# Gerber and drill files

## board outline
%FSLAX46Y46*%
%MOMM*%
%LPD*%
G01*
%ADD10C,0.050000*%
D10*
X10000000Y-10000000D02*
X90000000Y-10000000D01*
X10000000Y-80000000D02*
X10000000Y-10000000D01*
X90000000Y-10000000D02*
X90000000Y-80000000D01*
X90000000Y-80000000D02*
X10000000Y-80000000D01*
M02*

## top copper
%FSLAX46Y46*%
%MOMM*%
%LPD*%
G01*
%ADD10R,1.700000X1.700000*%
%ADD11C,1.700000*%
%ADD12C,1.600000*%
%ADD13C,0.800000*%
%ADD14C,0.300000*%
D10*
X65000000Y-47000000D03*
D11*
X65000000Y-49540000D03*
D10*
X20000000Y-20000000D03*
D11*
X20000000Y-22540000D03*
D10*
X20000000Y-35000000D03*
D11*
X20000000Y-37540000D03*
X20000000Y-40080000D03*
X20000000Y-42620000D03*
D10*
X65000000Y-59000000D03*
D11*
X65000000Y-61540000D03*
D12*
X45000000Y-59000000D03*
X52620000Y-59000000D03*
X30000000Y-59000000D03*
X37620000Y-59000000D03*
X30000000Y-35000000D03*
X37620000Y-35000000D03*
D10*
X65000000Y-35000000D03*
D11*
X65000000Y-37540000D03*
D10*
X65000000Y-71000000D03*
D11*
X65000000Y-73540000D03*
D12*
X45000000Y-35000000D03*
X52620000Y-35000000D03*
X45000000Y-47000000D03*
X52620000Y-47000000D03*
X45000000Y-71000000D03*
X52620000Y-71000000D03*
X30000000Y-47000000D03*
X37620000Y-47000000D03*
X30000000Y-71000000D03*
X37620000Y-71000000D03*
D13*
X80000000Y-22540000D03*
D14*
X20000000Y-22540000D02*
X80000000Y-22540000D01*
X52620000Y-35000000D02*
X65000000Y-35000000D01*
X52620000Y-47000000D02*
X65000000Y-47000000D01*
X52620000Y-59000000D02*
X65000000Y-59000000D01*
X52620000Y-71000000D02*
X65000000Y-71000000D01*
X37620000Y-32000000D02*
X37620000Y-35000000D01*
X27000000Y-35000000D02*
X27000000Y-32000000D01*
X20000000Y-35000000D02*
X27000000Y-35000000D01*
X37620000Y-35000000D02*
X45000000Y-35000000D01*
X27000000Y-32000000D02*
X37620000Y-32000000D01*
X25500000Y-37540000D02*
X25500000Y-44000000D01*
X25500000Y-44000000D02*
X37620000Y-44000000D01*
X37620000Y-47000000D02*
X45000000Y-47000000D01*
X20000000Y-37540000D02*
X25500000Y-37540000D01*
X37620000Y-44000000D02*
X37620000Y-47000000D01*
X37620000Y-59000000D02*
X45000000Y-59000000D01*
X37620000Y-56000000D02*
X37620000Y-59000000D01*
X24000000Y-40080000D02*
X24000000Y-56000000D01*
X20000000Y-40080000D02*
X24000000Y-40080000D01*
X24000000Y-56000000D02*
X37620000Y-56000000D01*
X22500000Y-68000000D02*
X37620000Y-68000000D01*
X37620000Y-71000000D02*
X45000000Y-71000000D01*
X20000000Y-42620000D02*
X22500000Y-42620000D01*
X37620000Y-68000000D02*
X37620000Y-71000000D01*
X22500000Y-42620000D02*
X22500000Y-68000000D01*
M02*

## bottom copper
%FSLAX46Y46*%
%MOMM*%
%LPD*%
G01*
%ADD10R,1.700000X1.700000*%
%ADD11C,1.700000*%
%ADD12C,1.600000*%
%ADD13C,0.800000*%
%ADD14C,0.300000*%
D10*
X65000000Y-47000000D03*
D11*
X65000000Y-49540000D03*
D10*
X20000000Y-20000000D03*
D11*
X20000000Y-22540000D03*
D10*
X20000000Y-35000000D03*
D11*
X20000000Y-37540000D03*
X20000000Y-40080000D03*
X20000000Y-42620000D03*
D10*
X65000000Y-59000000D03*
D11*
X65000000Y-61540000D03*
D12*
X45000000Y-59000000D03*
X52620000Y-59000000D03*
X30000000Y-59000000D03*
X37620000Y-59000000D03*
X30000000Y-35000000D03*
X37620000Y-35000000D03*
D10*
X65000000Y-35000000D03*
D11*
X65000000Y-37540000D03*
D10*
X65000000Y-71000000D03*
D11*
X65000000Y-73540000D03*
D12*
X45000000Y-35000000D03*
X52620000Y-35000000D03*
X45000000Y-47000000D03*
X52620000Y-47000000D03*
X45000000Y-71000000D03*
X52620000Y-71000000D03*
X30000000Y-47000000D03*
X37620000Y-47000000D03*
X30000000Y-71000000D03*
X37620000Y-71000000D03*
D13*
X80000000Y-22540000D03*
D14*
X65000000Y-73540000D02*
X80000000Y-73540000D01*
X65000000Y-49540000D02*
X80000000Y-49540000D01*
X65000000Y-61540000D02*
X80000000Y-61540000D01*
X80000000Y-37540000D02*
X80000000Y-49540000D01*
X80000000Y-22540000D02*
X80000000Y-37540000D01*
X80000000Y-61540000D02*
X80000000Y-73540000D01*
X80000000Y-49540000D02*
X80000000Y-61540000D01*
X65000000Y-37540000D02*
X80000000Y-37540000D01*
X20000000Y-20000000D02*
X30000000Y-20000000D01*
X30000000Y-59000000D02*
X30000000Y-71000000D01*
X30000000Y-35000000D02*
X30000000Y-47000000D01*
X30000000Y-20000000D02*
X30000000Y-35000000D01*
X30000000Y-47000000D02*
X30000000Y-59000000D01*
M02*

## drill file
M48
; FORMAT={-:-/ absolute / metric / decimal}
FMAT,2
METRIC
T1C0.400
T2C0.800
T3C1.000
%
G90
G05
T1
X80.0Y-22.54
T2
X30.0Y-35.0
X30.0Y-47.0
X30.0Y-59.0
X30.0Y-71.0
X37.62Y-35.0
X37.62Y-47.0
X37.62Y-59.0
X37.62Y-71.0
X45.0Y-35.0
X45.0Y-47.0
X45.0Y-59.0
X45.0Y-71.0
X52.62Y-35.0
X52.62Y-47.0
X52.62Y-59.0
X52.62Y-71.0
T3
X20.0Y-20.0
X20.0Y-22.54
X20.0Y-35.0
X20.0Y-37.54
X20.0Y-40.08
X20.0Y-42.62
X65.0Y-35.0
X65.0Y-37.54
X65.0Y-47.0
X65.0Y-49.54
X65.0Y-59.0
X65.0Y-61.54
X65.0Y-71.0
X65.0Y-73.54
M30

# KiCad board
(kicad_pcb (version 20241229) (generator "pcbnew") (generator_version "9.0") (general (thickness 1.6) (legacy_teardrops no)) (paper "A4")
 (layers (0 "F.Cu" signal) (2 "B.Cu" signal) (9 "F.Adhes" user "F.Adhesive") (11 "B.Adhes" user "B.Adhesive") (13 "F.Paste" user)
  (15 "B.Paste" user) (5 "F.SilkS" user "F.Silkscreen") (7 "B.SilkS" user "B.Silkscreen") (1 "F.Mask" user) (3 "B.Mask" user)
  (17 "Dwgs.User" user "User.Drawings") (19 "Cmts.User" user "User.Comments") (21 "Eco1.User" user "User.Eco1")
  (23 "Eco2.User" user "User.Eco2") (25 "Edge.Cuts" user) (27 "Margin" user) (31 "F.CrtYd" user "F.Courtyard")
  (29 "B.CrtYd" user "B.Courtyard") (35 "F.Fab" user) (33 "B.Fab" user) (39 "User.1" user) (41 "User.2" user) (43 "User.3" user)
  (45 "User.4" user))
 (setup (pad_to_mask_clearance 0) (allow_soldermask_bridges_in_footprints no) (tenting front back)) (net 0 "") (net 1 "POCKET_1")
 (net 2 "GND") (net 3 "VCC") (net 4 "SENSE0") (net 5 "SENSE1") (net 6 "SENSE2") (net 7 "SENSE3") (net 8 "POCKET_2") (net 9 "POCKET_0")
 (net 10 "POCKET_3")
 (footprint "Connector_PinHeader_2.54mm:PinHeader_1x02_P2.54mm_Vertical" (layer "F.Cu") (at 65 47)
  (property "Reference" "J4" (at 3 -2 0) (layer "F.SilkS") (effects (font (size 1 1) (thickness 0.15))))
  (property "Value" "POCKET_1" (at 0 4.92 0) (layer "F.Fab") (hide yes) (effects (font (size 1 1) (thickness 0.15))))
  (pad "1" thru_hole rect (at 0 0) (size 1.7 1.7) (drill 1) (layers "*.Cu" "*.Mask") (remove_unused_layers no) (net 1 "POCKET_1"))
  (pad "2" thru_hole circle (at 0 2.54) (size 1.7 1.7) (drill 1) (layers "*.Cu" "*.Mask") (remove_unused_layers no) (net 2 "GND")))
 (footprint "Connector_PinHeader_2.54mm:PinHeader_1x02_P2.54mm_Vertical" (layer "F.Cu") (at 20 20)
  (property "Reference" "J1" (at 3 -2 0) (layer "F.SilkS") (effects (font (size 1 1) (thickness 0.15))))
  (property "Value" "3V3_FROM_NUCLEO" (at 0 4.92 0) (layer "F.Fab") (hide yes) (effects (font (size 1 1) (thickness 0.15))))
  (pad "1" thru_hole rect (at 0 0) (size 1.7 1.7) (drill 1) (layers "*.Cu" "*.Mask") (remove_unused_layers no) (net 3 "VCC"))
  (pad "2" thru_hole circle (at 0 2.54) (size 1.7 1.7) (drill 1) (layers "*.Cu" "*.Mask") (remove_unused_layers no) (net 2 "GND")))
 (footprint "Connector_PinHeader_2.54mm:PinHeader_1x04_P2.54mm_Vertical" (layer "F.Cu") (at 20 35)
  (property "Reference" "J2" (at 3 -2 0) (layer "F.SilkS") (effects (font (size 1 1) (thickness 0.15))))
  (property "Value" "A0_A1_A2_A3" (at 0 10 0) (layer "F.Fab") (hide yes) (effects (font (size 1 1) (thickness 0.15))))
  (pad "1" thru_hole rect (at 0 0) (size 1.7 1.7) (drill 1) (layers "*.Cu" "*.Mask") (remove_unused_layers no) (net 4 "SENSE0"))
  (pad "2" thru_hole circle (at 0 2.54) (size 1.7 1.7) (drill 1) (layers "*.Cu" "*.Mask") (remove_unused_layers no) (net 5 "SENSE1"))
  (pad "3" thru_hole circle (at 0 5.08) (size 1.7 1.7) (drill 1) (layers "*.Cu" "*.Mask") (remove_unused_layers no) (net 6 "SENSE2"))
  (pad "4" thru_hole circle (at 0 7.62) (size 1.7 1.7) (drill 1) (layers "*.Cu" "*.Mask") (remove_unused_layers no) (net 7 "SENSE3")))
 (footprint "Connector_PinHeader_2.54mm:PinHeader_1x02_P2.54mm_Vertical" (layer "F.Cu") (at 65 59)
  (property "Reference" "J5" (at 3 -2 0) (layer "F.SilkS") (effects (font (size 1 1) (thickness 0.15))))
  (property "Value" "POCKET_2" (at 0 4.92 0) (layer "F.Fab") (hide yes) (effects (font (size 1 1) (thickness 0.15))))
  (pad "1" thru_hole rect (at 0 0) (size 1.7 1.7) (drill 1) (layers "*.Cu" "*.Mask") (remove_unused_layers no) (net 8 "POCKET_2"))
  (pad "2" thru_hole circle (at 0 2.54) (size 1.7 1.7) (drill 1) (layers "*.Cu" "*.Mask") (remove_unused_layers no) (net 2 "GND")))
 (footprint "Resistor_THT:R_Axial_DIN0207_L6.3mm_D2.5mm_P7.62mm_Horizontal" (layer "F.Cu") (at 45 59)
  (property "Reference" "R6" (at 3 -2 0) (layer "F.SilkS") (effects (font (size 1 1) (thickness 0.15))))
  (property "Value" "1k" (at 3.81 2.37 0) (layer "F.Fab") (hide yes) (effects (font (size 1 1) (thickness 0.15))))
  (pad "1" thru_hole circle (at 0 0) (size 1.6 1.6) (drill 0.8) (layers "*.Cu" "*.Mask") (remove_unused_layers no) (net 6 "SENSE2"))
  (pad "2" thru_hole circle (at 7.62 0) (size 1.6 1.6) (drill 0.8) (layers "*.Cu" "*.Mask") (remove_unused_layers no) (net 8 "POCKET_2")))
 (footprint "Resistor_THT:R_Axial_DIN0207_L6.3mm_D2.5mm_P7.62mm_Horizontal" (layer "F.Cu") (at 30 59)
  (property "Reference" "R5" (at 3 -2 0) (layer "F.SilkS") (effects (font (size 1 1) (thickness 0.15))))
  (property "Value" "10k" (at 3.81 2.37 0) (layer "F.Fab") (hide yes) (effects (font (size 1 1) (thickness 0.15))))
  (pad "1" thru_hole circle (at 0 0) (size 1.6 1.6) (drill 0.8) (layers "*.Cu" "*.Mask") (remove_unused_layers no) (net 3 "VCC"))
  (pad "2" thru_hole circle (at 7.62 0) (size 1.6 1.6) (drill 0.8) (layers "*.Cu" "*.Mask") (remove_unused_layers no) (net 6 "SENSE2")))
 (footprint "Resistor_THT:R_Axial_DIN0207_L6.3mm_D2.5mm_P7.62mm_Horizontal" (layer "F.Cu") (at 30 35)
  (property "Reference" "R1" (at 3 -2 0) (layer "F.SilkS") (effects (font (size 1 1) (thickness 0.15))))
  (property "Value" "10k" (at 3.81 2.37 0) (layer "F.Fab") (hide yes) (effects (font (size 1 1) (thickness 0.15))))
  (pad "1" thru_hole circle (at 0 0) (size 1.6 1.6) (drill 0.8) (layers "*.Cu" "*.Mask") (remove_unused_layers no) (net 3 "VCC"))
  (pad "2" thru_hole circle (at 7.62 0) (size 1.6 1.6) (drill 0.8) (layers "*.Cu" "*.Mask") (remove_unused_layers no) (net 4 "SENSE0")))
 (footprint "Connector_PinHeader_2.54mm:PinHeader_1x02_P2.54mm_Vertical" (layer "F.Cu") (at 65 35)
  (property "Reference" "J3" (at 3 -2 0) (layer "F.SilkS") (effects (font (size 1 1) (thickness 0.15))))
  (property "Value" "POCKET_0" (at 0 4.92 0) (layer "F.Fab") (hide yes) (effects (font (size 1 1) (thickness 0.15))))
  (pad "1" thru_hole rect (at 0 0) (size 1.7 1.7) (drill 1) (layers "*.Cu" "*.Mask") (remove_unused_layers no) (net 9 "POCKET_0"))
  (pad "2" thru_hole circle (at 0 2.54) (size 1.7 1.7) (drill 1) (layers "*.Cu" "*.Mask") (remove_unused_layers no) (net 2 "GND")))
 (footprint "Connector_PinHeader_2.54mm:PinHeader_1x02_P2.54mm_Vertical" (layer "F.Cu") (at 65 71)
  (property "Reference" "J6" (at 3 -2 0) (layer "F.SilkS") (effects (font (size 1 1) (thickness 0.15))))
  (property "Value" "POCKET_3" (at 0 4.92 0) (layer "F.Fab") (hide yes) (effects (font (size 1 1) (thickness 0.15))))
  (pad "1" thru_hole rect (at 0 0) (size 1.7 1.7) (drill 1) (layers "*.Cu" "*.Mask") (remove_unused_layers no) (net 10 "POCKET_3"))
  (pad "2" thru_hole circle (at 0 2.54) (size 1.7 1.7) (drill 1) (layers "*.Cu" "*.Mask") (remove_unused_layers no) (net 2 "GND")))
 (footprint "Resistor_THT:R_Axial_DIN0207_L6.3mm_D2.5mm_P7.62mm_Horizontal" (layer "F.Cu") (at 45 35)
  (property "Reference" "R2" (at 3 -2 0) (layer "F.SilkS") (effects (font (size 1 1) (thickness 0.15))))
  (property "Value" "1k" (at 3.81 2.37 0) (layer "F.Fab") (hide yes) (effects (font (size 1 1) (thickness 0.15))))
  (pad "1" thru_hole circle (at 0 0) (size 1.6 1.6) (drill 0.8) (layers "*.Cu" "*.Mask") (remove_unused_layers no) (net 4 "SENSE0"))
  (pad "2" thru_hole circle (at 7.62 0) (size 1.6 1.6) (drill 0.8) (layers "*.Cu" "*.Mask") (remove_unused_layers no) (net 9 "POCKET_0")))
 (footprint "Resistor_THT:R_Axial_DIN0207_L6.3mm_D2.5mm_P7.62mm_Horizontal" (layer "F.Cu") (at 45 47)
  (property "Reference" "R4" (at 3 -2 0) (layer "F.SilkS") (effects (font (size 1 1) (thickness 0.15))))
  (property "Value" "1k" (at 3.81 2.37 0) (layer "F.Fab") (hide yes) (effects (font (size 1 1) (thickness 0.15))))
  (pad "1" thru_hole circle (at 0 0) (size 1.6 1.6) (drill 0.8) (layers "*.Cu" "*.Mask") (remove_unused_layers no) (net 5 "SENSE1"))
  (pad "2" thru_hole circle (at 7.62 0) (size 1.6 1.6) (drill 0.8) (layers "*.Cu" "*.Mask") (remove_unused_layers no) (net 1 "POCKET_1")))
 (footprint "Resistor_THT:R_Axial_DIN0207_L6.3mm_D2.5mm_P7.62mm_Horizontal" (layer "F.Cu") (at 45 71)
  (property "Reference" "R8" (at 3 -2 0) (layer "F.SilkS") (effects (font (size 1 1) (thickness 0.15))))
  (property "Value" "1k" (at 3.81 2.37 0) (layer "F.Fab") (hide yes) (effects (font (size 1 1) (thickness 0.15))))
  (pad "1" thru_hole circle (at 0 0) (size 1.6 1.6) (drill 0.8) (layers "*.Cu" "*.Mask") (remove_unused_layers no) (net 7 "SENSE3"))
  (pad "2" thru_hole circle (at 7.62 0) (size 1.6 1.6) (drill 0.8) (layers "*.Cu" "*.Mask") (remove_unused_layers no) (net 10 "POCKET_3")))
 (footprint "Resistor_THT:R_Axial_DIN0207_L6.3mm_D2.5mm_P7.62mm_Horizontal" (layer "F.Cu") (at 30 47)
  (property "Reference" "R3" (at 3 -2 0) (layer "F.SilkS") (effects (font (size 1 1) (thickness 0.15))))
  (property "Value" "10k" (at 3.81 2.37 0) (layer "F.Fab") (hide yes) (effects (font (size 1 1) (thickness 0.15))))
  (pad "1" thru_hole circle (at 0 0) (size 1.6 1.6) (drill 0.8) (layers "*.Cu" "*.Mask") (remove_unused_layers no) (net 3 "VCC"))
  (pad "2" thru_hole circle (at 7.62 0) (size 1.6 1.6) (drill 0.8) (layers "*.Cu" "*.Mask") (remove_unused_layers no) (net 5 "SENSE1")))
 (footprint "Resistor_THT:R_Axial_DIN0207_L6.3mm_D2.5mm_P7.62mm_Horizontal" (layer "F.Cu") (at 30 71)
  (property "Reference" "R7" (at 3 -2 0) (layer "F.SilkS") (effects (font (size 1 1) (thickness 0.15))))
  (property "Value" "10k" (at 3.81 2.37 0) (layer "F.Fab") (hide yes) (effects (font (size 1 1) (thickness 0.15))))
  (pad "1" thru_hole circle (at 0 0) (size 1.6 1.6) (drill 0.8) (layers "*.Cu" "*.Mask") (remove_unused_layers no) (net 3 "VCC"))
  (pad "2" thru_hole circle (at 7.62 0) (size 1.6 1.6) (drill 0.8) (layers "*.Cu" "*.Mask") (remove_unused_layers no) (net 7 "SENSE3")))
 (gr_line (start 10 10) (end 90 10) (stroke (width 0.05) (type default)) (layer "Edge.Cuts"))
 (gr_line (start 10 80) (end 10 10) (stroke (width 0.05) (type default)) (layer "Edge.Cuts"))
 (gr_line (start 90 10) (end 90 80) (stroke (width 0.05) (type default)) (layer "Edge.Cuts"))
 (gr_line (start 90 80) (end 10 80) (stroke (width 0.05) (type default)) (layer "Edge.Cuts"))
 (segment (start 20 22.54) (end 80 22.54) (width 0.3) (layer "F.Cu") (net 2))
 (via (at 80 22.54) (size 0.8) (drill 0.4) (layers "F.Cu" "B.Cu") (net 2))
 (segment (start 65 73.54) (end 80 73.54) (width 0.3) (layer "B.Cu") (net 2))
 (segment (start 65 49.54) (end 80 49.54) (width 0.3) (layer "B.Cu") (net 2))
 (segment (start 65 61.54) (end 80 61.54) (width 0.3) (layer "B.Cu") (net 2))
 (segment (start 80 37.54) (end 80 49.54) (width 0.3) (layer "B.Cu") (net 2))
 (segment (start 80 22.54) (end 80 37.54) (width 0.3) (layer "B.Cu") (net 2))
 (segment (start 80 61.54) (end 80 73.54) (width 0.3) (layer "B.Cu") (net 2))
 (segment (start 80 49.54) (end 80 61.54) (width 0.3) (layer "B.Cu") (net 2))
 (segment (start 65 37.54) (end 80 37.54) (width 0.3) (layer "B.Cu") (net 2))
 (segment (start 52.62 35) (end 65 35) (width 0.3) (layer "F.Cu") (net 9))
 (segment (start 52.62 47) (end 65 47) (width 0.3) (layer "F.Cu") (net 1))
 (segment (start 52.62 59) (end 65 59) (width 0.3) (layer "F.Cu") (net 8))
 (segment (start 52.62 71) (end 65 71) (width 0.3) (layer "F.Cu") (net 10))
 (segment (start 37.62 32) (end 37.62 35) (width 0.3) (layer "F.Cu") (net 4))
 (segment (start 27 35) (end 27 32) (width 0.3) (layer "F.Cu") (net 4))
 (segment (start 20 35) (end 27 35) (width 0.3) (layer "F.Cu") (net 4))
 (segment (start 37.62 35) (end 45 35) (width 0.3) (layer "F.Cu") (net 4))
 (segment (start 27 32) (end 37.62 32) (width 0.3) (layer "F.Cu") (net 4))
 (segment (start 25.5 37.54) (end 25.5 44) (width 0.3) (layer "F.Cu") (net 5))
 (segment (start 25.5 44) (end 37.62 44) (width 0.3) (layer "F.Cu") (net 5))
 (segment (start 37.62 47) (end 45 47) (width 0.3) (layer "F.Cu") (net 5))
 (segment (start 20 37.54) (end 25.5 37.54) (width 0.3) (layer "F.Cu") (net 5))
 (segment (start 37.62 44) (end 37.62 47) (width 0.3) (layer "F.Cu") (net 5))
 (segment (start 37.62 59) (end 45 59) (width 0.3) (layer "F.Cu") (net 6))
 (segment (start 37.62 56) (end 37.62 59) (width 0.3) (layer "F.Cu") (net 6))
 (segment (start 24 40.08) (end 24 56) (width 0.3) (layer "F.Cu") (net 6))
 (segment (start 20 40.08) (end 24 40.08) (width 0.3) (layer "F.Cu") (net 6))
 (segment (start 24 56) (end 37.62 56) (width 0.3) (layer "F.Cu") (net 6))
 (segment (start 22.5 68) (end 37.62 68) (width 0.3) (layer "F.Cu") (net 7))
 (segment (start 37.62 71) (end 45 71) (width 0.3) (layer "F.Cu") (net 7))
 (segment (start 20 42.62) (end 22.5 42.62) (width 0.3) (layer "F.Cu") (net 7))
 (segment (start 37.62 68) (end 37.62 71) (width 0.3) (layer "F.Cu") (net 7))
 (segment (start 22.5 42.62) (end 22.5 68) (width 0.3) (layer "F.Cu") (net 7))
 (segment (start 20 20) (end 30 20) (width 0.3) (layer "B.Cu") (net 3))
 (segment (start 30 59) (end 30 71) (width 0.3) (layer "B.Cu") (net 3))
 (segment (start 30 35) (end 30 47) (width 0.3) (layer "B.Cu") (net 3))
 (segment (start 30 20) (end 30 35) (width 0.3) (layer "B.Cu") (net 3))
 (segment (start 30 47) (end 30 59) (width 0.3) (layer "B.Cu") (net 3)))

